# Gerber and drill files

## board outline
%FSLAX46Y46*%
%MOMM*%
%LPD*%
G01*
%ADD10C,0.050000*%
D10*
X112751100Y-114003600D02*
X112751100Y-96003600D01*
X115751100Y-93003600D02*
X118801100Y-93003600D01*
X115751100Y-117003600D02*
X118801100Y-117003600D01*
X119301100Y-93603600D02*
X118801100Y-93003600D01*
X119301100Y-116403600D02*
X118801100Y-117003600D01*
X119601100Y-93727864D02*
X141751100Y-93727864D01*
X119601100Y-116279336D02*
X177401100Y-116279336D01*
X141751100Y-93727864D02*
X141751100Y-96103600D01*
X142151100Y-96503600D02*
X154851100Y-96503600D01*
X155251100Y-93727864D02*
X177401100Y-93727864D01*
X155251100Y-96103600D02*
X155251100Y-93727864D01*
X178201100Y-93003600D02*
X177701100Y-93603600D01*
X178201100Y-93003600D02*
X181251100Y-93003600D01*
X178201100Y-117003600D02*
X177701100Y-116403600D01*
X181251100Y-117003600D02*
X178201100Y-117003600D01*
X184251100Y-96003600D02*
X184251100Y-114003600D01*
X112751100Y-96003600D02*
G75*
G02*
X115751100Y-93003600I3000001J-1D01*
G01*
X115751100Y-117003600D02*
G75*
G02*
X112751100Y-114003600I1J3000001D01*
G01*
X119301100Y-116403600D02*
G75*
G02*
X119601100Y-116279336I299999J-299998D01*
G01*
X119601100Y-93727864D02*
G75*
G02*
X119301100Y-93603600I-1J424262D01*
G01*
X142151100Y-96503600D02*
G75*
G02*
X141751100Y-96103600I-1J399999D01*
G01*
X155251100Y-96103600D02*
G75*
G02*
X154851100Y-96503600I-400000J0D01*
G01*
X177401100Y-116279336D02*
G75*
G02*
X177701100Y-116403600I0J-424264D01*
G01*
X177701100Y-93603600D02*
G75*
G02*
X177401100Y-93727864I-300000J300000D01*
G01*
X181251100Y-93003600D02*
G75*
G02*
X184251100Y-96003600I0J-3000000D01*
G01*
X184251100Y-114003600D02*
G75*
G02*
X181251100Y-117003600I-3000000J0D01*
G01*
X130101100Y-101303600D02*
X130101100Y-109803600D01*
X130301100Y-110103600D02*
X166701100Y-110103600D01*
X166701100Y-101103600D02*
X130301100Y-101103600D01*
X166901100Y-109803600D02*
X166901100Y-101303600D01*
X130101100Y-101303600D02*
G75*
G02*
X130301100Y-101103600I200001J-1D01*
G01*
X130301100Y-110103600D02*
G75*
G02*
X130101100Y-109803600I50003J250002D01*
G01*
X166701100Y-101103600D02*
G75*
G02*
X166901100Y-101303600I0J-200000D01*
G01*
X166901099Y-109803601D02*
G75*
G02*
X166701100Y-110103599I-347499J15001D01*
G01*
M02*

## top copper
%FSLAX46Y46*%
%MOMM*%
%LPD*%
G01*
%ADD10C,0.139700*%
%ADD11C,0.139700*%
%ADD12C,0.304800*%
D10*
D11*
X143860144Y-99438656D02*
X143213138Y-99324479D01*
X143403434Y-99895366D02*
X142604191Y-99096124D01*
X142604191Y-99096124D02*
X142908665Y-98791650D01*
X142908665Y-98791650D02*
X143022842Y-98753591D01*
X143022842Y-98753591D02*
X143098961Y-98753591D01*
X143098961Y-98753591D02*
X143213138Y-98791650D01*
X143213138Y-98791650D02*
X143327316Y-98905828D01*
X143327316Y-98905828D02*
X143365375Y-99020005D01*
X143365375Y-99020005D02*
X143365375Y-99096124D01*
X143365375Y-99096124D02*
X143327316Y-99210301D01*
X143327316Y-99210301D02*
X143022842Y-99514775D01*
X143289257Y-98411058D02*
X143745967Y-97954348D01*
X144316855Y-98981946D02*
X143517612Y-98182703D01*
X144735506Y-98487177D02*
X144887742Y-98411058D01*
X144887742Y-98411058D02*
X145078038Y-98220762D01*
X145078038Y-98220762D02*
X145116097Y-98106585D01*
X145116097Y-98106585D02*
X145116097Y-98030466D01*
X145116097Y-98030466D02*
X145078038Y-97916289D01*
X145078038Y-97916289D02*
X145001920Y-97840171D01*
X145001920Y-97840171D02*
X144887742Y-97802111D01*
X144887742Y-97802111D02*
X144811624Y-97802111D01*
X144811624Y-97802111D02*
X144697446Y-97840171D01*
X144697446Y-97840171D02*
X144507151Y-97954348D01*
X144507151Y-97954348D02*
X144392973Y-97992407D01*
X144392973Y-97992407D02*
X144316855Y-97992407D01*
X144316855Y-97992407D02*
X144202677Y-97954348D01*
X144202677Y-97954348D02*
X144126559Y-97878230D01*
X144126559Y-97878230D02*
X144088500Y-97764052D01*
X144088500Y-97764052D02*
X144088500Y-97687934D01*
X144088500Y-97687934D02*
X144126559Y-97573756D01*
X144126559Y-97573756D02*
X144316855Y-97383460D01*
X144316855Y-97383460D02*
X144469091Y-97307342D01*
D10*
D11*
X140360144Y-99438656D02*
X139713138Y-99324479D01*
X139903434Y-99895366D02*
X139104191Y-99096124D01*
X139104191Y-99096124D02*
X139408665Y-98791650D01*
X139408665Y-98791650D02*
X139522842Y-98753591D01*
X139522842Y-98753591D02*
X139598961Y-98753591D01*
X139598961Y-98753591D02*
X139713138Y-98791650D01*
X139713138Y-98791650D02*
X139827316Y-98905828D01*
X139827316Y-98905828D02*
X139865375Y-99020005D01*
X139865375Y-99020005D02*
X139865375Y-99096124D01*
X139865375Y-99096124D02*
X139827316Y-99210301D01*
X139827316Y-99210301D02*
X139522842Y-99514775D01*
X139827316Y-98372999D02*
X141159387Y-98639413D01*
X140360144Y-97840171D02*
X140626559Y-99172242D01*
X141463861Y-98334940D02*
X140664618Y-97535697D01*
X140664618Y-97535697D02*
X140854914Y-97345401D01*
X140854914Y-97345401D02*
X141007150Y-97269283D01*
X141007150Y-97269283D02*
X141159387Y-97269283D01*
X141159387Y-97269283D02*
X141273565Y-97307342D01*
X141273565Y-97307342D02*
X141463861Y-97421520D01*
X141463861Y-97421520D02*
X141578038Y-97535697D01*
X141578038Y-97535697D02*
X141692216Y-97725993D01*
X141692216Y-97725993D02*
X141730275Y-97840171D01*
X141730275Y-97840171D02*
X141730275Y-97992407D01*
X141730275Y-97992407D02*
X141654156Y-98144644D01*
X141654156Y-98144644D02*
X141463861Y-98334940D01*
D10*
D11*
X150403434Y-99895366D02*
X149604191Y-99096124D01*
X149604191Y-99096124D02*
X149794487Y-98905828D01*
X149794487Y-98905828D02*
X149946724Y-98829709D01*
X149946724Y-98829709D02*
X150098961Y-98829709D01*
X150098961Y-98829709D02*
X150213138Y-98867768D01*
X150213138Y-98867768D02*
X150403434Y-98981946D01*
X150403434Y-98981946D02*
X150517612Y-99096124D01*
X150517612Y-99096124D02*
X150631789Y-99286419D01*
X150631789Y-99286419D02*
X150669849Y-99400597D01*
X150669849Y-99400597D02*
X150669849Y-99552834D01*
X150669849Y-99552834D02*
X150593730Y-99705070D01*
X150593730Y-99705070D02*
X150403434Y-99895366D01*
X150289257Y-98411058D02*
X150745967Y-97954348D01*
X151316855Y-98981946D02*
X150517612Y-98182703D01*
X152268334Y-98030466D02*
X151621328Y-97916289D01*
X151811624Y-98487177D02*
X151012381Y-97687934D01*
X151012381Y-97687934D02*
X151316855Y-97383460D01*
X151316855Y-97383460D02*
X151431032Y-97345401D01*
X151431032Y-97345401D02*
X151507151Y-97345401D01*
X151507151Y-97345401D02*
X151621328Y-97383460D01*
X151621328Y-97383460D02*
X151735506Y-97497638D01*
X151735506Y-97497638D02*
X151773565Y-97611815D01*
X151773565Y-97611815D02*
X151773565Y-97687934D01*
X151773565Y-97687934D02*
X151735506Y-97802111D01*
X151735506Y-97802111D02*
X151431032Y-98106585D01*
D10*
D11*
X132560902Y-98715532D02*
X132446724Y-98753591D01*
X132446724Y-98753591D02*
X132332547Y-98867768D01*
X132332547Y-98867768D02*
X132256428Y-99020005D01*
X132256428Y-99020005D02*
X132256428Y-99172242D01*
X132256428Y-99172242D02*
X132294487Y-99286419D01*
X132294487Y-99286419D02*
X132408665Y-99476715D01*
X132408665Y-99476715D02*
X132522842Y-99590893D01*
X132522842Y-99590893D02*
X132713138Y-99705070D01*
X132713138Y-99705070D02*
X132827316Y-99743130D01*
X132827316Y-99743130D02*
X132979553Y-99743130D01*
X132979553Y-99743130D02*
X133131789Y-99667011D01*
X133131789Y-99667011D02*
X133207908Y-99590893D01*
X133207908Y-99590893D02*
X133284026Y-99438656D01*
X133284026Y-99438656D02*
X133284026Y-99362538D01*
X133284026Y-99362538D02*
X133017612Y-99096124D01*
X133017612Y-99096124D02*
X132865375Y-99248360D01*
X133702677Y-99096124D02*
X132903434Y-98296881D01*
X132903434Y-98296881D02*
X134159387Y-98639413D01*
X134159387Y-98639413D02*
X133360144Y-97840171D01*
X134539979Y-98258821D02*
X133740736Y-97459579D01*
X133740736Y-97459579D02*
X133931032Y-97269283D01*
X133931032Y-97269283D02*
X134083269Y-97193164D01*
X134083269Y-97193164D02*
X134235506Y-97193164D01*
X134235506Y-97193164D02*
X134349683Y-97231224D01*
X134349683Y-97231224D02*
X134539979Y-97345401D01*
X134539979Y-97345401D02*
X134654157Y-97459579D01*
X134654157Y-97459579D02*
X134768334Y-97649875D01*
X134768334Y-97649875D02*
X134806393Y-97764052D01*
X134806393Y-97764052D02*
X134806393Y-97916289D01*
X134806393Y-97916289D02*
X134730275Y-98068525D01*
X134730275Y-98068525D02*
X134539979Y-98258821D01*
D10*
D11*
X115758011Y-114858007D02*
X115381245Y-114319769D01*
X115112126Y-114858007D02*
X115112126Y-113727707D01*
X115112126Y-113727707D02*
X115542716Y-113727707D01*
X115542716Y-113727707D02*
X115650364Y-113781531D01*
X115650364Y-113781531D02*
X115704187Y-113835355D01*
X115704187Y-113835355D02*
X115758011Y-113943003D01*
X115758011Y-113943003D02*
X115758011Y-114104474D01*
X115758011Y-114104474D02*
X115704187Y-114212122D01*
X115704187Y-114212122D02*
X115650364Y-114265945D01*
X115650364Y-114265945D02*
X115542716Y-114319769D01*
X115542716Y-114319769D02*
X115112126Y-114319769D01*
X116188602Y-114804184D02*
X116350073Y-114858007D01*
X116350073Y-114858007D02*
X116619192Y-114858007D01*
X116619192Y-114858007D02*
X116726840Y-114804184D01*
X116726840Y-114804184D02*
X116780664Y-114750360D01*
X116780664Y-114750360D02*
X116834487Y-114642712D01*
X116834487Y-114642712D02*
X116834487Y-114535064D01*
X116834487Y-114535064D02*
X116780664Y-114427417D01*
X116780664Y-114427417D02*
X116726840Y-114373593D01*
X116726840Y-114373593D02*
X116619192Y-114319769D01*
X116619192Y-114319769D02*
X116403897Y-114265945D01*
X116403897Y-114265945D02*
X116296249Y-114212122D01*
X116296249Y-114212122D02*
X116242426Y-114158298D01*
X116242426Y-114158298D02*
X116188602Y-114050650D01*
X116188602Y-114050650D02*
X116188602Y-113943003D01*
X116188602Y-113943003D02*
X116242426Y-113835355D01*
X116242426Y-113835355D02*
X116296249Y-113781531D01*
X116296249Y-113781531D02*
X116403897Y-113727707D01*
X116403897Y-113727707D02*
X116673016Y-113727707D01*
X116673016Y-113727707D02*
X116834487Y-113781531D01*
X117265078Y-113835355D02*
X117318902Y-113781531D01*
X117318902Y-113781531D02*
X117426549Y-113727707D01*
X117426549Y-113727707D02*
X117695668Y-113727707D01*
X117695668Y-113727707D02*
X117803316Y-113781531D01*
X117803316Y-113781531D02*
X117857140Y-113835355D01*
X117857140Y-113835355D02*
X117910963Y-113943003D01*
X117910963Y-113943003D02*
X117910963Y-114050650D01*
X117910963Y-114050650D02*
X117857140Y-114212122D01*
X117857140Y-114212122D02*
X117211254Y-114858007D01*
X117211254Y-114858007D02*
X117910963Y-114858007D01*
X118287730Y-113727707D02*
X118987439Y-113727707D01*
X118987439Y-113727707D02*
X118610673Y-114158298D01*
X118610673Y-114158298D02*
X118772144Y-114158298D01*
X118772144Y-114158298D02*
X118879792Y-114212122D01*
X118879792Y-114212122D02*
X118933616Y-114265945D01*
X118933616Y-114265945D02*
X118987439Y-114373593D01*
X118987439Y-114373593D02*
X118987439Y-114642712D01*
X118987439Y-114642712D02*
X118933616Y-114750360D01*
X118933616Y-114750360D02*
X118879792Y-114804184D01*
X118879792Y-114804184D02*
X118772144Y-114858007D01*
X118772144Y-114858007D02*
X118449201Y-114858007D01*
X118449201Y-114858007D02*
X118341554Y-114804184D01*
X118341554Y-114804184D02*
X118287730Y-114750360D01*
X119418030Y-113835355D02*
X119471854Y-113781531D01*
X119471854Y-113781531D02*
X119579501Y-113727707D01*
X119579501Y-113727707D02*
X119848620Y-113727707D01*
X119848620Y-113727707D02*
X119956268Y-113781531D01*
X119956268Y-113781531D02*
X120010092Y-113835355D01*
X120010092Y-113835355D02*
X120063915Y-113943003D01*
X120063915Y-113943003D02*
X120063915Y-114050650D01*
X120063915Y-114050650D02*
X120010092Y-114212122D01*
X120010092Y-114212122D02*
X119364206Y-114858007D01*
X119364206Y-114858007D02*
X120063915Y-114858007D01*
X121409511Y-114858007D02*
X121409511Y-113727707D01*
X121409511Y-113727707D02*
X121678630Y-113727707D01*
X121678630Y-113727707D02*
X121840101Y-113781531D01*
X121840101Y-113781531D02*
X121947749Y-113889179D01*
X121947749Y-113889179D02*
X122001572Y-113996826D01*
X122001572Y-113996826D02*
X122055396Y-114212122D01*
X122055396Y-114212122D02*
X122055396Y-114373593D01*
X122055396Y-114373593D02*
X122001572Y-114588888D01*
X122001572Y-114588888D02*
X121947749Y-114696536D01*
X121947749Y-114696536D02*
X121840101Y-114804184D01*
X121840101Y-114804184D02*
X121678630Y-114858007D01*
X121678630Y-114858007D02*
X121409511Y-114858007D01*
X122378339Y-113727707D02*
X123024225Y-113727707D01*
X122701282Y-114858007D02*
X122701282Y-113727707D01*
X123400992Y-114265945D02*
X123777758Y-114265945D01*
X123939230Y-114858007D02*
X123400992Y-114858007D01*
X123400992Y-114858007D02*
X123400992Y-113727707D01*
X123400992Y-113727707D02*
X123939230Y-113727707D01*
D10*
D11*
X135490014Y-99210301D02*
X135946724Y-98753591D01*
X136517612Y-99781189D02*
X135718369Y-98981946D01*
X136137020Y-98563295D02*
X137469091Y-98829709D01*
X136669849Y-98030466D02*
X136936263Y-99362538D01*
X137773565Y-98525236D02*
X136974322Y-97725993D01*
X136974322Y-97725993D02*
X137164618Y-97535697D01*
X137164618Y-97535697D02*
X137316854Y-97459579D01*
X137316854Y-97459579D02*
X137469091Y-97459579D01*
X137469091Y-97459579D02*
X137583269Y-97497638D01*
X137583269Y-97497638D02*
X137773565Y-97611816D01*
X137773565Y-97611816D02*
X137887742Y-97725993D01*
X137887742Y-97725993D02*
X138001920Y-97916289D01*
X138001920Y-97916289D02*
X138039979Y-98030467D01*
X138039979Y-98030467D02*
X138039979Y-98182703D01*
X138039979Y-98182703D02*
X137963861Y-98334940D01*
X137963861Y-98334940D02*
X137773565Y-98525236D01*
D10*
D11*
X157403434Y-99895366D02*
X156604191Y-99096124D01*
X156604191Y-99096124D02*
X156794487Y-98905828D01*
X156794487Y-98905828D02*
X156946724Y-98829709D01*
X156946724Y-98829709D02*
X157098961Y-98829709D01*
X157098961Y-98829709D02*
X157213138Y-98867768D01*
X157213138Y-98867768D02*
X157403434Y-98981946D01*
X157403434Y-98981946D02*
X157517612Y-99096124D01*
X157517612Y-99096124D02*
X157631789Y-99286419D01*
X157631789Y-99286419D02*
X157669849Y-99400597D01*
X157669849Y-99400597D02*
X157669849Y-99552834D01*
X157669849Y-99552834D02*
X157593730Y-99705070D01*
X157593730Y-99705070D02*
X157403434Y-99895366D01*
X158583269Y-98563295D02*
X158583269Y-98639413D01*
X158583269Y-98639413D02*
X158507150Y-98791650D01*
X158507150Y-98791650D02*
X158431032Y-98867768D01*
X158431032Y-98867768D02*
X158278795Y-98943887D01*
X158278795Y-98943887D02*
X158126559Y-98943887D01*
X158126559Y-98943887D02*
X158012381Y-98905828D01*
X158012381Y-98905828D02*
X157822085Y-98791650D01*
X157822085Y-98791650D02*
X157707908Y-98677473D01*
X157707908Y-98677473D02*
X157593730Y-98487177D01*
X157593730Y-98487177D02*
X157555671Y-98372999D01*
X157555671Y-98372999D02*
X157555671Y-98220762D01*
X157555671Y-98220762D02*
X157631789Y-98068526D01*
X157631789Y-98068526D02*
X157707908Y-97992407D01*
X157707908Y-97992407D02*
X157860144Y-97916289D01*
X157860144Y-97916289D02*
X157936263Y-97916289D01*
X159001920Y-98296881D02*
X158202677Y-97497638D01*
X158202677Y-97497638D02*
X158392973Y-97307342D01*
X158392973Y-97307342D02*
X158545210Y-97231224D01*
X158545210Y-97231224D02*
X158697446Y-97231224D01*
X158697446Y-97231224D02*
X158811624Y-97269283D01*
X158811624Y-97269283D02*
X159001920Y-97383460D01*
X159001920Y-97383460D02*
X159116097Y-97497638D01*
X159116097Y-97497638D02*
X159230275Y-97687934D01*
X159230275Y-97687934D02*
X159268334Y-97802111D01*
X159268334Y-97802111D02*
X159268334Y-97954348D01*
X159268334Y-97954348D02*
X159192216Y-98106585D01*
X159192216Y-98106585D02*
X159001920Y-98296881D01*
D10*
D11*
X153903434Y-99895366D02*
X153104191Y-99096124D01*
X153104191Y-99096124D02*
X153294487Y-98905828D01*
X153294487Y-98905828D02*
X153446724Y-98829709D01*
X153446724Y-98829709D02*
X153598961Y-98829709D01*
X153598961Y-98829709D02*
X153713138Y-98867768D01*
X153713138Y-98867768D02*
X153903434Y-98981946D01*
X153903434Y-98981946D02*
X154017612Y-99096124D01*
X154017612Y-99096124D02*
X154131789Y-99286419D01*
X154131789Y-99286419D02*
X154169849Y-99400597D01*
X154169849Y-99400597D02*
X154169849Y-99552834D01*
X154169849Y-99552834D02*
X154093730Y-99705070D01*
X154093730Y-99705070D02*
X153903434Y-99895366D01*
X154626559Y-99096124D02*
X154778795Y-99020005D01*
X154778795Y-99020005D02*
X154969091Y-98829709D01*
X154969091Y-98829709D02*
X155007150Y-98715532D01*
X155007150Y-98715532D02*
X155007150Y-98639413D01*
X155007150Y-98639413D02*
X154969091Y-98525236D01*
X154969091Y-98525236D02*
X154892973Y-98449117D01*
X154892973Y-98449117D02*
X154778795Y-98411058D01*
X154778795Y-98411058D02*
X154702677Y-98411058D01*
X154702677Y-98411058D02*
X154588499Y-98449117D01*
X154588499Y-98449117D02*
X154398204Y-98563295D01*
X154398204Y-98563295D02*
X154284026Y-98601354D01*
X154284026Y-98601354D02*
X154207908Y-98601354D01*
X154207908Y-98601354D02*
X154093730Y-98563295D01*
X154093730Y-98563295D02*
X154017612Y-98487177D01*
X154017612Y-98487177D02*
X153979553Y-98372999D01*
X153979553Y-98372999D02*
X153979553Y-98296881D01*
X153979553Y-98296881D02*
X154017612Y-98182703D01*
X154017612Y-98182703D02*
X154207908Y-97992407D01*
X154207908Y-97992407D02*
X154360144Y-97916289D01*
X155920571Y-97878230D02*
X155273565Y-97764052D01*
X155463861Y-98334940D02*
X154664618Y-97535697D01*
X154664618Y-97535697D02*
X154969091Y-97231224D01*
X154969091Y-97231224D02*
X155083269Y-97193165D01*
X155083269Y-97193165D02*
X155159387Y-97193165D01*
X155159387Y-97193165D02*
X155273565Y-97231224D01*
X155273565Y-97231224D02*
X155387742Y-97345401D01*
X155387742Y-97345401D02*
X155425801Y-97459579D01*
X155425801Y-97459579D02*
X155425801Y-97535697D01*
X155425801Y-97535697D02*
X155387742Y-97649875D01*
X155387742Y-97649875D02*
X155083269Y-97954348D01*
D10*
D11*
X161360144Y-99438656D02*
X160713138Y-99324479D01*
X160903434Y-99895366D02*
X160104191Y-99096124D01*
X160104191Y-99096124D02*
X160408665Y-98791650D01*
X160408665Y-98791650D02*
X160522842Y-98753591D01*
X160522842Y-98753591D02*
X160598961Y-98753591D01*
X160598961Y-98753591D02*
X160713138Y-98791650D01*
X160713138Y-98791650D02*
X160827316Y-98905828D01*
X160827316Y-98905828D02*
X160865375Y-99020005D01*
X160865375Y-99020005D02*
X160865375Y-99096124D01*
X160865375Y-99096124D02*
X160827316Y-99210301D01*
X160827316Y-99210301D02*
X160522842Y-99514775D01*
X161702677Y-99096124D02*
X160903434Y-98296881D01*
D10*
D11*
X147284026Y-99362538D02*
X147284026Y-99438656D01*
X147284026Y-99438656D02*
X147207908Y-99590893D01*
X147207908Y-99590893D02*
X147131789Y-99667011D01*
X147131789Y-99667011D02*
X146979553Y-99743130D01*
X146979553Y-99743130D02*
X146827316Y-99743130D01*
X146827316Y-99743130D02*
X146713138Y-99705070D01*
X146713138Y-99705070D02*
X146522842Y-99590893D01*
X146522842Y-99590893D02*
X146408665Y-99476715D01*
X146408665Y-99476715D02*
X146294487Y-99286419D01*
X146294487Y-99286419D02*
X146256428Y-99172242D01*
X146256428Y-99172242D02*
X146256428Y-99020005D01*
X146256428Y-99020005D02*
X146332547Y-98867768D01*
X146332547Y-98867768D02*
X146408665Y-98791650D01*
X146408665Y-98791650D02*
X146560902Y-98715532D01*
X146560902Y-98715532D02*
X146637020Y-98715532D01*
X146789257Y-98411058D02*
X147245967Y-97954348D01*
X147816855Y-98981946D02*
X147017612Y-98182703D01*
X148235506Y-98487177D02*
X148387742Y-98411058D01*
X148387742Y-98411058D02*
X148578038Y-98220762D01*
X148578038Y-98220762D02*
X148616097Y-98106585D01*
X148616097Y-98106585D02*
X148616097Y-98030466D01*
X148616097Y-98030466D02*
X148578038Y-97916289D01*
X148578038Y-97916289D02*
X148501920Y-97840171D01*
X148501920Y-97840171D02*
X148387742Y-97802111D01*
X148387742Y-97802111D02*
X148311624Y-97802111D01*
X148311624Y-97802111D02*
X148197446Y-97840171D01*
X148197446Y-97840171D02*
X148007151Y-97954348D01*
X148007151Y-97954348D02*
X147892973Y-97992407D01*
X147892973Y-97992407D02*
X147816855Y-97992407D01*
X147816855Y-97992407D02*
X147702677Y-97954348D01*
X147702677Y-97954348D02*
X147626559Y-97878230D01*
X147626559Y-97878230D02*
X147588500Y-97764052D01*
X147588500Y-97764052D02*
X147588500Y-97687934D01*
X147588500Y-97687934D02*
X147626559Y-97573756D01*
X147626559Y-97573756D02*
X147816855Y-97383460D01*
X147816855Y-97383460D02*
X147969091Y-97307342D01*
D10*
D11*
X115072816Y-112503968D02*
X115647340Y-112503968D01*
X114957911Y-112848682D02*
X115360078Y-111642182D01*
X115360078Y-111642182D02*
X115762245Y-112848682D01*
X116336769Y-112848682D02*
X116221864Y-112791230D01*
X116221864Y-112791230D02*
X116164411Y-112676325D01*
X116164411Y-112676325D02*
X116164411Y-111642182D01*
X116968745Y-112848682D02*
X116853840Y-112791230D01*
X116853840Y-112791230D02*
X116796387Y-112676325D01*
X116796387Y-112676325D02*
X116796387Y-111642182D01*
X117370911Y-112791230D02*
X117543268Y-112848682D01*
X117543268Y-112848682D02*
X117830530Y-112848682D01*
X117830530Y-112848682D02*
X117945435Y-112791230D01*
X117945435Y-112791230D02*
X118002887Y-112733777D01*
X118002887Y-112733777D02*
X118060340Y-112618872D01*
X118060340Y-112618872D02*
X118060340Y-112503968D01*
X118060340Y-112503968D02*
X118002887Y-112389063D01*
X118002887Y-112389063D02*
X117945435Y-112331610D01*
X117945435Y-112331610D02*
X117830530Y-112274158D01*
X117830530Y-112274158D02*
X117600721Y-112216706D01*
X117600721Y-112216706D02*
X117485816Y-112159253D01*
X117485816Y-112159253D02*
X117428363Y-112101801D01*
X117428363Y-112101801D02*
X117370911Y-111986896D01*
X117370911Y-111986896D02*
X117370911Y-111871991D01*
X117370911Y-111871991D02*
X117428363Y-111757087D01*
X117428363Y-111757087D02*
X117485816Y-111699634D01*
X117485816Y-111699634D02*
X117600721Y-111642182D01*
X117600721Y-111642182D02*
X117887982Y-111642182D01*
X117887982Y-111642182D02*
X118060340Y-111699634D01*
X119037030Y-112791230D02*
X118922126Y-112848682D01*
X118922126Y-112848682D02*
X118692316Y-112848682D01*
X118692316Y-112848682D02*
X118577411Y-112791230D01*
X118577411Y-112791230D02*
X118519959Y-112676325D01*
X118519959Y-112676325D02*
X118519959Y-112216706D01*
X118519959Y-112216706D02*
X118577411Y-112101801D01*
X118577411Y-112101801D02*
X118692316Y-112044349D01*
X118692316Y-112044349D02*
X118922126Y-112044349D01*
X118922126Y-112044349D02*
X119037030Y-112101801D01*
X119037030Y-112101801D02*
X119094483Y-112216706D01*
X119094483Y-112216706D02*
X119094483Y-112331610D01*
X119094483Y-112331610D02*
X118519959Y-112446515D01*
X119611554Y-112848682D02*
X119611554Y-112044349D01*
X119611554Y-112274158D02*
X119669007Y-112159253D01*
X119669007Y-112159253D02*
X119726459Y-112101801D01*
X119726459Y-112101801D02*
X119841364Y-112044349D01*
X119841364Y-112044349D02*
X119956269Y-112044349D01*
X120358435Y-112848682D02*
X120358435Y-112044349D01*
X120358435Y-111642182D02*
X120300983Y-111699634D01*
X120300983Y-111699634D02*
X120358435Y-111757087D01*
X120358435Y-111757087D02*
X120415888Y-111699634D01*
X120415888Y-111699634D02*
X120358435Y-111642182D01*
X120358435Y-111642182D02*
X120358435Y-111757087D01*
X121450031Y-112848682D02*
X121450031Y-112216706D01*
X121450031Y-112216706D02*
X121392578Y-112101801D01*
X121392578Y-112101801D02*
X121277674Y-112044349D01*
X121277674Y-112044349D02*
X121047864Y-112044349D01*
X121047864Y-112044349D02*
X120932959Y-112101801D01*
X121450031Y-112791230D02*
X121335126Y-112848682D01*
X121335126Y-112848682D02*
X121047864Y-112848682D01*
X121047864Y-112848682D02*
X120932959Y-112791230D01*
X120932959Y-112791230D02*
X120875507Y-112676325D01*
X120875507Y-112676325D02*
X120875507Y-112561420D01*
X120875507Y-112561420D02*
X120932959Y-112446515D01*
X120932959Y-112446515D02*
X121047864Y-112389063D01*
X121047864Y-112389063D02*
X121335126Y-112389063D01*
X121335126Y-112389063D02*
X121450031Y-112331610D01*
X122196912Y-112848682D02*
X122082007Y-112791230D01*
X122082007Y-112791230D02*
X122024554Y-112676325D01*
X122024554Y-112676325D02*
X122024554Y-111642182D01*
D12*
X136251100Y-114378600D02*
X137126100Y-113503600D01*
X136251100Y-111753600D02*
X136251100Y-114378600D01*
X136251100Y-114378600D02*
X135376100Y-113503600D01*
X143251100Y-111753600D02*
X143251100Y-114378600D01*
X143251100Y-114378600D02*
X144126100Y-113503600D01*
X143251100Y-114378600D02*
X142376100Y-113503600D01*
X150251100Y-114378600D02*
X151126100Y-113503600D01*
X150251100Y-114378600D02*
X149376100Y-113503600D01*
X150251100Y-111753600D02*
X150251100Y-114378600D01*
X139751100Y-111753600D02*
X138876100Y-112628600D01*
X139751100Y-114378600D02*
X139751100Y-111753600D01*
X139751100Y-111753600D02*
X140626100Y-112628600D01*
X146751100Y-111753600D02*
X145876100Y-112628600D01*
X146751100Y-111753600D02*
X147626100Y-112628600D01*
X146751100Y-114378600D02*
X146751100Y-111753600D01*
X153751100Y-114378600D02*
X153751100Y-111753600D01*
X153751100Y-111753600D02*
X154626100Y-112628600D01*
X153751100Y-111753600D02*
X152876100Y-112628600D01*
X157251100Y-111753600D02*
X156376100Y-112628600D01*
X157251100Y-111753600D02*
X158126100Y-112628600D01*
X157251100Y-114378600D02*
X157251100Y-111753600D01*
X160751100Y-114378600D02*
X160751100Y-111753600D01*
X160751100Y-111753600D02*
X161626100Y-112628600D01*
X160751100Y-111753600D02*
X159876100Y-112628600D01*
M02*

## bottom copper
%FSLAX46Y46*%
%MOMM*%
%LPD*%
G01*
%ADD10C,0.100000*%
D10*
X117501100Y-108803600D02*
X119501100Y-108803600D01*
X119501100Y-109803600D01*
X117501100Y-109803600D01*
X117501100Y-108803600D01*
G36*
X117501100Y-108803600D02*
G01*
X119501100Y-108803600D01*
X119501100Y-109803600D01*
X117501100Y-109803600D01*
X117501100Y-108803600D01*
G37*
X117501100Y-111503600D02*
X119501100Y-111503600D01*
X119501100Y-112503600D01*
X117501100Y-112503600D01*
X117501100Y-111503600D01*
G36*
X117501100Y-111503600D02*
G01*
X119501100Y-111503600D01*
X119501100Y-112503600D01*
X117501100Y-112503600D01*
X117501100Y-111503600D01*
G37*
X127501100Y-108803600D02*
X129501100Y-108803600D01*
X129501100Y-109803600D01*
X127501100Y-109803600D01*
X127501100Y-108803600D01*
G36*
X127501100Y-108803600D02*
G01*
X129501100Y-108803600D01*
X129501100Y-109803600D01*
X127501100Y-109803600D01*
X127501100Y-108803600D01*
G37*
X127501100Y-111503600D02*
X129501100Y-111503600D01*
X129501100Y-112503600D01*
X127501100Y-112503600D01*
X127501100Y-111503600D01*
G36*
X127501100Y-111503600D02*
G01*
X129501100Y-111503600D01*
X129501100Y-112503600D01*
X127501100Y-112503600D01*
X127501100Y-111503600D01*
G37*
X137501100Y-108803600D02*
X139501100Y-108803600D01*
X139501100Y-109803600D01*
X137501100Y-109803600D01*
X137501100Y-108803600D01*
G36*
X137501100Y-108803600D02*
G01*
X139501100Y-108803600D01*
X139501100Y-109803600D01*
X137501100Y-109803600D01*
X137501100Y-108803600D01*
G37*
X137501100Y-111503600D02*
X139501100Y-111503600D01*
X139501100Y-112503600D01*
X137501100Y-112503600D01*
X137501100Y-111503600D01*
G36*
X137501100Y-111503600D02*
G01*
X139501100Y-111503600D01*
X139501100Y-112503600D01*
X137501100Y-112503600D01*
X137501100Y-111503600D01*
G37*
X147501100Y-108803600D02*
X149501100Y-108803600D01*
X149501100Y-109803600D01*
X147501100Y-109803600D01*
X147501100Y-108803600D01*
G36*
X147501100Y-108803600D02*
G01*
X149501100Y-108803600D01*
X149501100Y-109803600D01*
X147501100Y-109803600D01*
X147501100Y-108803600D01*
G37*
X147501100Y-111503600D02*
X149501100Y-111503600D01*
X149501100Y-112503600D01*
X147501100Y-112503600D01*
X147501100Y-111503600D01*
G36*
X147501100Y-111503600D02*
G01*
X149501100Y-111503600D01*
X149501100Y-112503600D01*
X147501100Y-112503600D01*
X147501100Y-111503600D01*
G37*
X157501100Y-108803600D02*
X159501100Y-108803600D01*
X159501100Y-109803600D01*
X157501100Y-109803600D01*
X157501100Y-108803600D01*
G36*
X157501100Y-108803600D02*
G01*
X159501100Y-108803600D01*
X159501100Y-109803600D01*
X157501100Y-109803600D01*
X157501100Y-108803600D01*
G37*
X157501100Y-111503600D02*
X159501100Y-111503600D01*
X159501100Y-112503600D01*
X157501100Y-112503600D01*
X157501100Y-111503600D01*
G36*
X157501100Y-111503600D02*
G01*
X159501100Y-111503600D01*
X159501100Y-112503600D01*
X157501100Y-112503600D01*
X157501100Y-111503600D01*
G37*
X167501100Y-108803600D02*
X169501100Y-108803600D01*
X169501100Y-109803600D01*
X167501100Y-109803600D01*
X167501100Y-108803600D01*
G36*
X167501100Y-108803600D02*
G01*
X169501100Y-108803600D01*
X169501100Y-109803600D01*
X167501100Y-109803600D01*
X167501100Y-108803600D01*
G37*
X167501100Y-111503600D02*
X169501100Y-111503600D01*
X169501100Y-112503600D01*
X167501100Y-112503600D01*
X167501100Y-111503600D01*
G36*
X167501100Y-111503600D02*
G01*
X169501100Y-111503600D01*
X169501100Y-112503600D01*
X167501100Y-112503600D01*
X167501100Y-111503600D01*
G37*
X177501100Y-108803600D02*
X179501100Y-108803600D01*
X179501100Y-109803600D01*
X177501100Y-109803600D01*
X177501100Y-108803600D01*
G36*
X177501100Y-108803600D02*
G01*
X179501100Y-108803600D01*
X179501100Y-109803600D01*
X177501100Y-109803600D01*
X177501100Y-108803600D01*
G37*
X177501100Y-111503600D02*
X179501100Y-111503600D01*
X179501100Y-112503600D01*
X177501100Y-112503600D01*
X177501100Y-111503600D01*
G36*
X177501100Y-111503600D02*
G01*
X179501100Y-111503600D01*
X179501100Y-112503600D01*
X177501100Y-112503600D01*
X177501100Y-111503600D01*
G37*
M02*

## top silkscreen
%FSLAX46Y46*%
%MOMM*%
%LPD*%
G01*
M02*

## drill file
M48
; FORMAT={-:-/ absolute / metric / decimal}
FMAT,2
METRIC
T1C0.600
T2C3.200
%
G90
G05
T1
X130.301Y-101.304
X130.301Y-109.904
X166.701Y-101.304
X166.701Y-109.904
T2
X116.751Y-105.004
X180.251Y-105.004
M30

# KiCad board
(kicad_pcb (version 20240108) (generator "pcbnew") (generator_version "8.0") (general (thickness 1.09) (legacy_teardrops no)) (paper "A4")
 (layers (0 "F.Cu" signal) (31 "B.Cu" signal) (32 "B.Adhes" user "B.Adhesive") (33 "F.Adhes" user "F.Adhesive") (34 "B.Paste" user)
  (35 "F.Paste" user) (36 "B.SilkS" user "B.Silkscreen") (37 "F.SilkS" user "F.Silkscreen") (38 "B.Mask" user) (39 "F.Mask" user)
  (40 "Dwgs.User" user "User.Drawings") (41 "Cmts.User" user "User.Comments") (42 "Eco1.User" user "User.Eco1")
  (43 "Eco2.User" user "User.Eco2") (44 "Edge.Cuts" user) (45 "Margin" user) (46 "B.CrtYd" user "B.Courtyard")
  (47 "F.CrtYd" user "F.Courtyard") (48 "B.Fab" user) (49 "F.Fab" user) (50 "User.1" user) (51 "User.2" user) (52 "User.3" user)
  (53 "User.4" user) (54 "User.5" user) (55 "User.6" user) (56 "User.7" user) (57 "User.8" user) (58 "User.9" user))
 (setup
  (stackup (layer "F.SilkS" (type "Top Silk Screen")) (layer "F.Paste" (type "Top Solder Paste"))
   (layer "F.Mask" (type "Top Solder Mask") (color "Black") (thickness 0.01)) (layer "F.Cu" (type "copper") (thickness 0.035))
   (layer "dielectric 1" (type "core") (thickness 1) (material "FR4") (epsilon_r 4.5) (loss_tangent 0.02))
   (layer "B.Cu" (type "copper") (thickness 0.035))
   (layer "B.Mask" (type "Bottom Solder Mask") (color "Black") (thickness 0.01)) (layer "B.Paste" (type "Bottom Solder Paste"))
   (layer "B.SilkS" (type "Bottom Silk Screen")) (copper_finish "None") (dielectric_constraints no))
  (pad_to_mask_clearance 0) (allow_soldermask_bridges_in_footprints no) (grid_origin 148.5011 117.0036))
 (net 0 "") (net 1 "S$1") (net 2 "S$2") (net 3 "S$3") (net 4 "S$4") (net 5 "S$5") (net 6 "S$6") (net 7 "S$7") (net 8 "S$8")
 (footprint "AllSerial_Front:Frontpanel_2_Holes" (layer "F.Cu") (at 148.5011 117.0036)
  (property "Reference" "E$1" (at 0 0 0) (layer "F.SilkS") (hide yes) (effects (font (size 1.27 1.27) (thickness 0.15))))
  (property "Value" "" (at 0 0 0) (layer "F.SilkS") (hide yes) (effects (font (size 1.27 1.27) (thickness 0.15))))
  (fp_rect (start -31 -8.2) (end -29 -7.2) (stroke (width 0.1) (type solid)) (fill solid) (layer "B.Cu"))
  (fp_rect (start -31 -5.5) (end -29 -4.5) (stroke (width 0.1) (type solid)) (fill solid) (layer "B.Cu"))
  (fp_rect (start -21 -8.2) (end -19 -7.2) (stroke (width 0.1) (type solid)) (fill solid) (layer "B.Cu"))
  (fp_rect (start -21 -5.5) (end -19 -4.5) (stroke (width 0.1) (type solid)) (fill solid) (layer "B.Cu"))
  (fp_rect (start -11 -8.2) (end -9 -7.2) (stroke (width 0.1) (type solid)) (fill solid) (layer "B.Cu"))
  (fp_rect (start -11 -5.5) (end -9 -4.5) (stroke (width 0.1) (type solid)) (fill solid) (layer "B.Cu"))
  (fp_rect (start -1 -8.2) (end 1 -7.2) (stroke (width 0.1) (type solid)) (fill solid) (layer "B.Cu"))
  (fp_rect (start -1 -5.5) (end 1 -4.5) (stroke (width 0.1) (type solid)) (fill solid) (layer "B.Cu"))
  (fp_rect (start 9 -8.2) (end 11 -7.2) (stroke (width 0.1) (type solid)) (fill solid) (layer "B.Cu"))
  (fp_rect (start 9 -5.5) (end 11 -4.5) (stroke (width 0.1) (type solid)) (fill solid) (layer "B.Cu"))
  (fp_rect (start 19 -8.2) (end 21 -7.2) (stroke (width 0.1) (type solid)) (fill solid) (layer "B.Cu"))
  (fp_rect (start 19 -5.5) (end 21 -4.5) (stroke (width 0.1) (type solid)) (fill solid) (layer "B.Cu"))
  (fp_rect (start 29 -8.2) (end 31 -7.2) (stroke (width 0.1) (type solid)) (fill solid) (layer "B.Cu"))
  (fp_rect (start 29 -5.5) (end 31 -4.5) (stroke (width 0.1) (type solid)) (fill solid) (layer "B.Cu"))
  (fp_line (start -35.75 -3) (end -35.75 -21) (stroke (width 0.05) (type solid)) (layer "Edge.Cuts"))
  (fp_line (start -32.75 -24) (end -29.7 -24) (stroke (width 0.05) (type solid)) (layer "Edge.Cuts"))
  (fp_line (start -32.75 0) (end -29.7 0) (stroke (width 0.05) (type default)) (layer "Edge.Cuts"))
  (fp_line (start -29.2 -23.4) (end -29.7 -24) (stroke (width 0.05) (type default)) (layer "Edge.Cuts"))
  (fp_line (start -29.2 -0.6) (end -29.7 0) (stroke (width 0.05) (type default)) (layer "Edge.Cuts"))
  (fp_line (start -28.9 -23.275736) (end -6.75 -23.275736) (stroke (width 0.05) (type default)) (layer "Edge.Cuts"))
  (fp_line (start -28.9 -0.724264) (end 28.9 -0.724264) (stroke (width 0.05) (type default)) (layer "Edge.Cuts"))
  (fp_line (start -6.75 -23.275736) (end -6.75 -20.9) (stroke (width 0.05) (type solid)) (layer "Edge.Cuts"))
  (fp_line (start -6.35 -20.5) (end 6.35 -20.5) (stroke (width 0.05) (type solid)) (layer "Edge.Cuts"))
  (fp_line (start 6.75 -23.275736) (end 28.9 -23.275736) (stroke (width 0.05) (type default)) (layer "Edge.Cuts"))
  (fp_line (start 6.75 -20.9) (end 6.75 -23.275736) (stroke (width 0.05) (type solid)) (layer "Edge.Cuts"))
  (fp_line (start 29.7 -24) (end 29.2 -23.4) (stroke (width 0.05) (type default)) (layer "Edge.Cuts"))
  (fp_line (start 29.7 -24) (end 32.75 -24) (stroke (width 0.05) (type solid)) (layer "Edge.Cuts"))
  (fp_line (start 29.7 0) (end 29.2 -0.6) (stroke (width 0.05) (type default)) (layer "Edge.Cuts"))
  (fp_line (start 32.75 0) (end 29.7 0) (stroke (width 0.05) (type default)) (layer "Edge.Cuts"))
  (fp_line (start 35.75 -21) (end 35.75 -3) (stroke (width 0.05) (type solid)) (layer "Edge.Cuts"))
  (fp_arc (start -35.75 -21) (mid -34.87132 -23.12132) (end -32.75 -24) (stroke (width 0.05) (type solid)) (layer "Edge.Cuts"))
  (fp_arc (start -32.75 0) (mid -34.87132 -0.87868) (end -35.75 -3) (stroke (width 0.05) (type solid)) (layer "Edge.Cuts"))
  (fp_arc (start -29.2 -0.6) (mid -29.062359 -0.691969) (end -28.9 -0.724264) (stroke (width 0.05) (type default)) (layer "Edge.Cuts"))
  (fp_arc (start -28.9 -23.275736) (mid -29.062359 -23.308031) (end -29.2 -23.4) (stroke (width 0.05) (type default)) (layer "Edge.Cuts"))
  (fp_arc (start -6.35 -20.5) (mid -6.632843 -20.617157) (end -6.75 -20.9) (stroke (width 0.05) (type solid)) (layer "Edge.Cuts"))
  (fp_arc (start 6.75 -20.9) (mid 6.632843 -20.617157) (end 6.35 -20.5) (stroke (width 0.05) (type solid)) (layer "Edge.Cuts"))
  (fp_arc (start 28.9 -0.724264) (mid 29.062359 -0.691969) (end 29.2 -0.6) (stroke (width 0.05) (type default)) (layer "Edge.Cuts"))
  (fp_arc (start 29.2 -23.4) (mid 29.062359 -23.308031) (end 28.9 -23.275736) (stroke (width 0.05) (type default)) (layer "Edge.Cuts"))
  (fp_arc (start 32.75 -24) (mid 34.87132 -23.12132) (end 35.75 -21) (stroke (width 0.05) (type solid)) (layer "Edge.Cuts"))
  (fp_arc (start 35.75 -3) (mid 34.87132 -0.87868) (end 32.75 0) (stroke (width 0.05) (type solid)) (layer "Edge.Cuts"))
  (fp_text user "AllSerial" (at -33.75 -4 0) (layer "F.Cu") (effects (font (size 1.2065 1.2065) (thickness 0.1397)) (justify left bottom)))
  (pad "" np_thru_hole circle (at -31.75 -12) (size 3.2 3.2) (drill 3.2) (layers "*.Cu" "*.Mask"))
  (pad "" np_thru_hole circle (at 31.75 -12) (size 3.2 3.2) (drill 3.2) (layers "*.Cu" "*.Mask")))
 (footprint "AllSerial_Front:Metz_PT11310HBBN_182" (layer "F.Cu") (at 148.5011 117.0036)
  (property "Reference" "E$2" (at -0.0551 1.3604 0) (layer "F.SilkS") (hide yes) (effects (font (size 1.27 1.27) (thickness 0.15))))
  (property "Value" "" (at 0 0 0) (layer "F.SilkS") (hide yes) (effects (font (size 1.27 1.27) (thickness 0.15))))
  (fp_line (start -18.4 -15.7) (end -18.4 -7.2) (stroke (width 0.05) (type solid)) (layer "Edge.Cuts"))
  (fp_line (start -18.2 -6.9) (end 18.2 -6.9) (stroke (width 0.05) (type solid)) (layer "Edge.Cuts"))
  (fp_line (start 18.2 -15.9) (end -18.2 -15.9) (stroke (width 0.05) (type solid)) (layer "Edge.Cuts"))
  (fp_line (start 18.4 -7.2) (end 18.4 -15.7) (stroke (width 0.05) (type solid)) (layer "Edge.Cuts"))
  (fp_arc (start -18.4 -15.7) (mid -18.341421 -15.841421) (end -18.2 -15.9) (stroke (width 0.05) (type solid)) (layer "Edge.Cuts"))
  (fp_arc (start -18.2 -6.9) (mid -18.362131 -7.008579) (end -18.4 -7.2) (stroke (width 0.05) (type solid)) (layer "Edge.Cuts"))
  (fp_arc (start 18.2 -15.9) (mid 18.341421 -15.841421) (end 18.4 -15.7) (stroke (width 0.05) (type solid)) (layer "Edge.Cuts"))
  (fp_arc (start 18.399999 -7.199999) (mid 18.341906 -7.022062) (end 18.2 -6.9) (stroke (width 0.05) (type solid)) (layer "Edge.Cuts"))
  (pad "" np_thru_hole circle (at -18.2 -15.7) (size 0.6 0.6) (drill 0.6) (layers "*.Cu" "*.Mask"))
  (pad "" np_thru_hole circle (at -18.2 -7.1) (size 0.6 0.6) (drill 0.6) (layers "*.Cu" "*.Mask"))
  (pad "" np_thru_hole circle (at 18.2 -15.7) (size 0.6 0.6) (drill 0.6) (layers "*.Cu" "*.Mask"))
  (pad "" np_thru_hole circle (at 18.2 -7.1) (size 0.6 0.6) (drill 0.6) (layers "*.Cu" "*.Mask")))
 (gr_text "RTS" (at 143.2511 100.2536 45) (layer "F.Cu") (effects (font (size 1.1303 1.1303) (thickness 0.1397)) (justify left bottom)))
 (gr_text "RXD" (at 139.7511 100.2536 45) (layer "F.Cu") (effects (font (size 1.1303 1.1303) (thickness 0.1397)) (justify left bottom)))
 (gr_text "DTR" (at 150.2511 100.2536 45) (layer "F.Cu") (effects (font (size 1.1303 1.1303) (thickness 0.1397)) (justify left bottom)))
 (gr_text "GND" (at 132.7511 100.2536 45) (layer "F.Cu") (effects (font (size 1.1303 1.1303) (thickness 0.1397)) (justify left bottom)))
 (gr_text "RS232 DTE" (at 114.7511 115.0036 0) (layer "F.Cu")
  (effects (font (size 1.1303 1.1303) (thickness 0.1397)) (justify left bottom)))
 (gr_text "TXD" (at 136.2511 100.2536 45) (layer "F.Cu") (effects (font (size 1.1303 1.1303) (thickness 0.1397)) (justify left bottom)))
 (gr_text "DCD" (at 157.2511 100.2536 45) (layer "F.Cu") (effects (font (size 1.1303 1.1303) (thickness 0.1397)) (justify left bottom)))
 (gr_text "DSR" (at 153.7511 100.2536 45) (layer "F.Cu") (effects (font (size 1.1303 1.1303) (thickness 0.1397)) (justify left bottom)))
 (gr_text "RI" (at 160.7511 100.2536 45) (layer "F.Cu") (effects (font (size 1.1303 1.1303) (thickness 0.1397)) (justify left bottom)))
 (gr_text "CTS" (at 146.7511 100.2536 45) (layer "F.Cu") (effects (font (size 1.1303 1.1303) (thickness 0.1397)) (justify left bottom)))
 (segment (start 136.2511 114.3786) (end 137.1261 113.5036) (width 0.3048) (layer "F.Cu") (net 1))
 (segment (start 136.2511 111.7536) (end 136.2511 114.3786) (width 0.3048) (layer "F.Cu") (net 1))
 (segment (start 136.2511 114.3786) (end 135.3761 113.5036) (width 0.3048) (layer "F.Cu") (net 1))
 (segment (start 143.2511 111.7536) (end 143.2511 114.3786) (width 0.3048) (layer "F.Cu") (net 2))
 (segment (start 143.2511 114.3786) (end 144.1261 113.5036) (width 0.3048) (layer "F.Cu") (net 2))
 (segment (start 143.2511 114.3786) (end 142.3761 113.5036) (width 0.3048) (layer "F.Cu") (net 2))
 (segment (start 150.2511 114.3786) (end 151.1261 113.5036) (width 0.3048) (layer "F.Cu") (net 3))
 (segment (start 150.2511 114.3786) (end 149.3761 113.5036) (width 0.3048) (layer "F.Cu") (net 3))
 (segment (start 150.2511 111.7536) (end 150.2511 114.3786) (width 0.3048) (layer "F.Cu") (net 3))
 (segment (start 139.7511 111.7536) (end 138.8761 112.6286) (width 0.3048) (layer "F.Cu") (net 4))
 (segment (start 139.7511 114.3786) (end 139.7511 111.7536) (width 0.3048) (layer "F.Cu") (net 4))
 (segment (start 139.7511 111.7536) (end 140.6261 112.6286) (width 0.3048) (layer "F.Cu") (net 4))
 (segment (start 146.7511 111.7536) (end 145.8761 112.6286) (width 0.3048) (layer "F.Cu") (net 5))
 (segment (start 146.7511 111.7536) (end 147.6261 112.6286) (width 0.3048) (layer "F.Cu") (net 5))
 (segment (start 146.7511 114.3786) (end 146.7511 111.7536) (width 0.3048) (layer "F.Cu") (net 5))
 (segment (start 153.7511 114.3786) (end 153.7511 111.7536) (width 0.3048) (layer "F.Cu") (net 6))
 (segment (start 153.7511 111.7536) (end 154.6261 112.6286) (width 0.3048) (layer "F.Cu") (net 6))
 (segment (start 153.7511 111.7536) (end 152.8761 112.6286) (width 0.3048) (layer "F.Cu") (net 6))
 (segment (start 157.2511 111.7536) (end 156.3761 112.6286) (width 0.3048) (layer "F.Cu") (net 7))
 (segment (start 157.2511 111.7536) (end 158.1261 112.6286) (width 0.3048) (layer "F.Cu") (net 7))
 (segment (start 157.2511 114.3786) (end 157.2511 111.7536) (width 0.3048) (layer "F.Cu") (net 7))
 (segment (start 160.7511 114.3786) (end 160.7511 111.7536) (width 0.3048) (layer "F.Cu") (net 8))
 (segment (start 160.7511 111.7536) (end 161.6261 112.6286) (width 0.3048) (layer "F.Cu") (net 8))
 (segment (start 160.7511 111.7536) (end 159.8761 112.6286) (width 0.3048) (layer "F.Cu") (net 8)))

